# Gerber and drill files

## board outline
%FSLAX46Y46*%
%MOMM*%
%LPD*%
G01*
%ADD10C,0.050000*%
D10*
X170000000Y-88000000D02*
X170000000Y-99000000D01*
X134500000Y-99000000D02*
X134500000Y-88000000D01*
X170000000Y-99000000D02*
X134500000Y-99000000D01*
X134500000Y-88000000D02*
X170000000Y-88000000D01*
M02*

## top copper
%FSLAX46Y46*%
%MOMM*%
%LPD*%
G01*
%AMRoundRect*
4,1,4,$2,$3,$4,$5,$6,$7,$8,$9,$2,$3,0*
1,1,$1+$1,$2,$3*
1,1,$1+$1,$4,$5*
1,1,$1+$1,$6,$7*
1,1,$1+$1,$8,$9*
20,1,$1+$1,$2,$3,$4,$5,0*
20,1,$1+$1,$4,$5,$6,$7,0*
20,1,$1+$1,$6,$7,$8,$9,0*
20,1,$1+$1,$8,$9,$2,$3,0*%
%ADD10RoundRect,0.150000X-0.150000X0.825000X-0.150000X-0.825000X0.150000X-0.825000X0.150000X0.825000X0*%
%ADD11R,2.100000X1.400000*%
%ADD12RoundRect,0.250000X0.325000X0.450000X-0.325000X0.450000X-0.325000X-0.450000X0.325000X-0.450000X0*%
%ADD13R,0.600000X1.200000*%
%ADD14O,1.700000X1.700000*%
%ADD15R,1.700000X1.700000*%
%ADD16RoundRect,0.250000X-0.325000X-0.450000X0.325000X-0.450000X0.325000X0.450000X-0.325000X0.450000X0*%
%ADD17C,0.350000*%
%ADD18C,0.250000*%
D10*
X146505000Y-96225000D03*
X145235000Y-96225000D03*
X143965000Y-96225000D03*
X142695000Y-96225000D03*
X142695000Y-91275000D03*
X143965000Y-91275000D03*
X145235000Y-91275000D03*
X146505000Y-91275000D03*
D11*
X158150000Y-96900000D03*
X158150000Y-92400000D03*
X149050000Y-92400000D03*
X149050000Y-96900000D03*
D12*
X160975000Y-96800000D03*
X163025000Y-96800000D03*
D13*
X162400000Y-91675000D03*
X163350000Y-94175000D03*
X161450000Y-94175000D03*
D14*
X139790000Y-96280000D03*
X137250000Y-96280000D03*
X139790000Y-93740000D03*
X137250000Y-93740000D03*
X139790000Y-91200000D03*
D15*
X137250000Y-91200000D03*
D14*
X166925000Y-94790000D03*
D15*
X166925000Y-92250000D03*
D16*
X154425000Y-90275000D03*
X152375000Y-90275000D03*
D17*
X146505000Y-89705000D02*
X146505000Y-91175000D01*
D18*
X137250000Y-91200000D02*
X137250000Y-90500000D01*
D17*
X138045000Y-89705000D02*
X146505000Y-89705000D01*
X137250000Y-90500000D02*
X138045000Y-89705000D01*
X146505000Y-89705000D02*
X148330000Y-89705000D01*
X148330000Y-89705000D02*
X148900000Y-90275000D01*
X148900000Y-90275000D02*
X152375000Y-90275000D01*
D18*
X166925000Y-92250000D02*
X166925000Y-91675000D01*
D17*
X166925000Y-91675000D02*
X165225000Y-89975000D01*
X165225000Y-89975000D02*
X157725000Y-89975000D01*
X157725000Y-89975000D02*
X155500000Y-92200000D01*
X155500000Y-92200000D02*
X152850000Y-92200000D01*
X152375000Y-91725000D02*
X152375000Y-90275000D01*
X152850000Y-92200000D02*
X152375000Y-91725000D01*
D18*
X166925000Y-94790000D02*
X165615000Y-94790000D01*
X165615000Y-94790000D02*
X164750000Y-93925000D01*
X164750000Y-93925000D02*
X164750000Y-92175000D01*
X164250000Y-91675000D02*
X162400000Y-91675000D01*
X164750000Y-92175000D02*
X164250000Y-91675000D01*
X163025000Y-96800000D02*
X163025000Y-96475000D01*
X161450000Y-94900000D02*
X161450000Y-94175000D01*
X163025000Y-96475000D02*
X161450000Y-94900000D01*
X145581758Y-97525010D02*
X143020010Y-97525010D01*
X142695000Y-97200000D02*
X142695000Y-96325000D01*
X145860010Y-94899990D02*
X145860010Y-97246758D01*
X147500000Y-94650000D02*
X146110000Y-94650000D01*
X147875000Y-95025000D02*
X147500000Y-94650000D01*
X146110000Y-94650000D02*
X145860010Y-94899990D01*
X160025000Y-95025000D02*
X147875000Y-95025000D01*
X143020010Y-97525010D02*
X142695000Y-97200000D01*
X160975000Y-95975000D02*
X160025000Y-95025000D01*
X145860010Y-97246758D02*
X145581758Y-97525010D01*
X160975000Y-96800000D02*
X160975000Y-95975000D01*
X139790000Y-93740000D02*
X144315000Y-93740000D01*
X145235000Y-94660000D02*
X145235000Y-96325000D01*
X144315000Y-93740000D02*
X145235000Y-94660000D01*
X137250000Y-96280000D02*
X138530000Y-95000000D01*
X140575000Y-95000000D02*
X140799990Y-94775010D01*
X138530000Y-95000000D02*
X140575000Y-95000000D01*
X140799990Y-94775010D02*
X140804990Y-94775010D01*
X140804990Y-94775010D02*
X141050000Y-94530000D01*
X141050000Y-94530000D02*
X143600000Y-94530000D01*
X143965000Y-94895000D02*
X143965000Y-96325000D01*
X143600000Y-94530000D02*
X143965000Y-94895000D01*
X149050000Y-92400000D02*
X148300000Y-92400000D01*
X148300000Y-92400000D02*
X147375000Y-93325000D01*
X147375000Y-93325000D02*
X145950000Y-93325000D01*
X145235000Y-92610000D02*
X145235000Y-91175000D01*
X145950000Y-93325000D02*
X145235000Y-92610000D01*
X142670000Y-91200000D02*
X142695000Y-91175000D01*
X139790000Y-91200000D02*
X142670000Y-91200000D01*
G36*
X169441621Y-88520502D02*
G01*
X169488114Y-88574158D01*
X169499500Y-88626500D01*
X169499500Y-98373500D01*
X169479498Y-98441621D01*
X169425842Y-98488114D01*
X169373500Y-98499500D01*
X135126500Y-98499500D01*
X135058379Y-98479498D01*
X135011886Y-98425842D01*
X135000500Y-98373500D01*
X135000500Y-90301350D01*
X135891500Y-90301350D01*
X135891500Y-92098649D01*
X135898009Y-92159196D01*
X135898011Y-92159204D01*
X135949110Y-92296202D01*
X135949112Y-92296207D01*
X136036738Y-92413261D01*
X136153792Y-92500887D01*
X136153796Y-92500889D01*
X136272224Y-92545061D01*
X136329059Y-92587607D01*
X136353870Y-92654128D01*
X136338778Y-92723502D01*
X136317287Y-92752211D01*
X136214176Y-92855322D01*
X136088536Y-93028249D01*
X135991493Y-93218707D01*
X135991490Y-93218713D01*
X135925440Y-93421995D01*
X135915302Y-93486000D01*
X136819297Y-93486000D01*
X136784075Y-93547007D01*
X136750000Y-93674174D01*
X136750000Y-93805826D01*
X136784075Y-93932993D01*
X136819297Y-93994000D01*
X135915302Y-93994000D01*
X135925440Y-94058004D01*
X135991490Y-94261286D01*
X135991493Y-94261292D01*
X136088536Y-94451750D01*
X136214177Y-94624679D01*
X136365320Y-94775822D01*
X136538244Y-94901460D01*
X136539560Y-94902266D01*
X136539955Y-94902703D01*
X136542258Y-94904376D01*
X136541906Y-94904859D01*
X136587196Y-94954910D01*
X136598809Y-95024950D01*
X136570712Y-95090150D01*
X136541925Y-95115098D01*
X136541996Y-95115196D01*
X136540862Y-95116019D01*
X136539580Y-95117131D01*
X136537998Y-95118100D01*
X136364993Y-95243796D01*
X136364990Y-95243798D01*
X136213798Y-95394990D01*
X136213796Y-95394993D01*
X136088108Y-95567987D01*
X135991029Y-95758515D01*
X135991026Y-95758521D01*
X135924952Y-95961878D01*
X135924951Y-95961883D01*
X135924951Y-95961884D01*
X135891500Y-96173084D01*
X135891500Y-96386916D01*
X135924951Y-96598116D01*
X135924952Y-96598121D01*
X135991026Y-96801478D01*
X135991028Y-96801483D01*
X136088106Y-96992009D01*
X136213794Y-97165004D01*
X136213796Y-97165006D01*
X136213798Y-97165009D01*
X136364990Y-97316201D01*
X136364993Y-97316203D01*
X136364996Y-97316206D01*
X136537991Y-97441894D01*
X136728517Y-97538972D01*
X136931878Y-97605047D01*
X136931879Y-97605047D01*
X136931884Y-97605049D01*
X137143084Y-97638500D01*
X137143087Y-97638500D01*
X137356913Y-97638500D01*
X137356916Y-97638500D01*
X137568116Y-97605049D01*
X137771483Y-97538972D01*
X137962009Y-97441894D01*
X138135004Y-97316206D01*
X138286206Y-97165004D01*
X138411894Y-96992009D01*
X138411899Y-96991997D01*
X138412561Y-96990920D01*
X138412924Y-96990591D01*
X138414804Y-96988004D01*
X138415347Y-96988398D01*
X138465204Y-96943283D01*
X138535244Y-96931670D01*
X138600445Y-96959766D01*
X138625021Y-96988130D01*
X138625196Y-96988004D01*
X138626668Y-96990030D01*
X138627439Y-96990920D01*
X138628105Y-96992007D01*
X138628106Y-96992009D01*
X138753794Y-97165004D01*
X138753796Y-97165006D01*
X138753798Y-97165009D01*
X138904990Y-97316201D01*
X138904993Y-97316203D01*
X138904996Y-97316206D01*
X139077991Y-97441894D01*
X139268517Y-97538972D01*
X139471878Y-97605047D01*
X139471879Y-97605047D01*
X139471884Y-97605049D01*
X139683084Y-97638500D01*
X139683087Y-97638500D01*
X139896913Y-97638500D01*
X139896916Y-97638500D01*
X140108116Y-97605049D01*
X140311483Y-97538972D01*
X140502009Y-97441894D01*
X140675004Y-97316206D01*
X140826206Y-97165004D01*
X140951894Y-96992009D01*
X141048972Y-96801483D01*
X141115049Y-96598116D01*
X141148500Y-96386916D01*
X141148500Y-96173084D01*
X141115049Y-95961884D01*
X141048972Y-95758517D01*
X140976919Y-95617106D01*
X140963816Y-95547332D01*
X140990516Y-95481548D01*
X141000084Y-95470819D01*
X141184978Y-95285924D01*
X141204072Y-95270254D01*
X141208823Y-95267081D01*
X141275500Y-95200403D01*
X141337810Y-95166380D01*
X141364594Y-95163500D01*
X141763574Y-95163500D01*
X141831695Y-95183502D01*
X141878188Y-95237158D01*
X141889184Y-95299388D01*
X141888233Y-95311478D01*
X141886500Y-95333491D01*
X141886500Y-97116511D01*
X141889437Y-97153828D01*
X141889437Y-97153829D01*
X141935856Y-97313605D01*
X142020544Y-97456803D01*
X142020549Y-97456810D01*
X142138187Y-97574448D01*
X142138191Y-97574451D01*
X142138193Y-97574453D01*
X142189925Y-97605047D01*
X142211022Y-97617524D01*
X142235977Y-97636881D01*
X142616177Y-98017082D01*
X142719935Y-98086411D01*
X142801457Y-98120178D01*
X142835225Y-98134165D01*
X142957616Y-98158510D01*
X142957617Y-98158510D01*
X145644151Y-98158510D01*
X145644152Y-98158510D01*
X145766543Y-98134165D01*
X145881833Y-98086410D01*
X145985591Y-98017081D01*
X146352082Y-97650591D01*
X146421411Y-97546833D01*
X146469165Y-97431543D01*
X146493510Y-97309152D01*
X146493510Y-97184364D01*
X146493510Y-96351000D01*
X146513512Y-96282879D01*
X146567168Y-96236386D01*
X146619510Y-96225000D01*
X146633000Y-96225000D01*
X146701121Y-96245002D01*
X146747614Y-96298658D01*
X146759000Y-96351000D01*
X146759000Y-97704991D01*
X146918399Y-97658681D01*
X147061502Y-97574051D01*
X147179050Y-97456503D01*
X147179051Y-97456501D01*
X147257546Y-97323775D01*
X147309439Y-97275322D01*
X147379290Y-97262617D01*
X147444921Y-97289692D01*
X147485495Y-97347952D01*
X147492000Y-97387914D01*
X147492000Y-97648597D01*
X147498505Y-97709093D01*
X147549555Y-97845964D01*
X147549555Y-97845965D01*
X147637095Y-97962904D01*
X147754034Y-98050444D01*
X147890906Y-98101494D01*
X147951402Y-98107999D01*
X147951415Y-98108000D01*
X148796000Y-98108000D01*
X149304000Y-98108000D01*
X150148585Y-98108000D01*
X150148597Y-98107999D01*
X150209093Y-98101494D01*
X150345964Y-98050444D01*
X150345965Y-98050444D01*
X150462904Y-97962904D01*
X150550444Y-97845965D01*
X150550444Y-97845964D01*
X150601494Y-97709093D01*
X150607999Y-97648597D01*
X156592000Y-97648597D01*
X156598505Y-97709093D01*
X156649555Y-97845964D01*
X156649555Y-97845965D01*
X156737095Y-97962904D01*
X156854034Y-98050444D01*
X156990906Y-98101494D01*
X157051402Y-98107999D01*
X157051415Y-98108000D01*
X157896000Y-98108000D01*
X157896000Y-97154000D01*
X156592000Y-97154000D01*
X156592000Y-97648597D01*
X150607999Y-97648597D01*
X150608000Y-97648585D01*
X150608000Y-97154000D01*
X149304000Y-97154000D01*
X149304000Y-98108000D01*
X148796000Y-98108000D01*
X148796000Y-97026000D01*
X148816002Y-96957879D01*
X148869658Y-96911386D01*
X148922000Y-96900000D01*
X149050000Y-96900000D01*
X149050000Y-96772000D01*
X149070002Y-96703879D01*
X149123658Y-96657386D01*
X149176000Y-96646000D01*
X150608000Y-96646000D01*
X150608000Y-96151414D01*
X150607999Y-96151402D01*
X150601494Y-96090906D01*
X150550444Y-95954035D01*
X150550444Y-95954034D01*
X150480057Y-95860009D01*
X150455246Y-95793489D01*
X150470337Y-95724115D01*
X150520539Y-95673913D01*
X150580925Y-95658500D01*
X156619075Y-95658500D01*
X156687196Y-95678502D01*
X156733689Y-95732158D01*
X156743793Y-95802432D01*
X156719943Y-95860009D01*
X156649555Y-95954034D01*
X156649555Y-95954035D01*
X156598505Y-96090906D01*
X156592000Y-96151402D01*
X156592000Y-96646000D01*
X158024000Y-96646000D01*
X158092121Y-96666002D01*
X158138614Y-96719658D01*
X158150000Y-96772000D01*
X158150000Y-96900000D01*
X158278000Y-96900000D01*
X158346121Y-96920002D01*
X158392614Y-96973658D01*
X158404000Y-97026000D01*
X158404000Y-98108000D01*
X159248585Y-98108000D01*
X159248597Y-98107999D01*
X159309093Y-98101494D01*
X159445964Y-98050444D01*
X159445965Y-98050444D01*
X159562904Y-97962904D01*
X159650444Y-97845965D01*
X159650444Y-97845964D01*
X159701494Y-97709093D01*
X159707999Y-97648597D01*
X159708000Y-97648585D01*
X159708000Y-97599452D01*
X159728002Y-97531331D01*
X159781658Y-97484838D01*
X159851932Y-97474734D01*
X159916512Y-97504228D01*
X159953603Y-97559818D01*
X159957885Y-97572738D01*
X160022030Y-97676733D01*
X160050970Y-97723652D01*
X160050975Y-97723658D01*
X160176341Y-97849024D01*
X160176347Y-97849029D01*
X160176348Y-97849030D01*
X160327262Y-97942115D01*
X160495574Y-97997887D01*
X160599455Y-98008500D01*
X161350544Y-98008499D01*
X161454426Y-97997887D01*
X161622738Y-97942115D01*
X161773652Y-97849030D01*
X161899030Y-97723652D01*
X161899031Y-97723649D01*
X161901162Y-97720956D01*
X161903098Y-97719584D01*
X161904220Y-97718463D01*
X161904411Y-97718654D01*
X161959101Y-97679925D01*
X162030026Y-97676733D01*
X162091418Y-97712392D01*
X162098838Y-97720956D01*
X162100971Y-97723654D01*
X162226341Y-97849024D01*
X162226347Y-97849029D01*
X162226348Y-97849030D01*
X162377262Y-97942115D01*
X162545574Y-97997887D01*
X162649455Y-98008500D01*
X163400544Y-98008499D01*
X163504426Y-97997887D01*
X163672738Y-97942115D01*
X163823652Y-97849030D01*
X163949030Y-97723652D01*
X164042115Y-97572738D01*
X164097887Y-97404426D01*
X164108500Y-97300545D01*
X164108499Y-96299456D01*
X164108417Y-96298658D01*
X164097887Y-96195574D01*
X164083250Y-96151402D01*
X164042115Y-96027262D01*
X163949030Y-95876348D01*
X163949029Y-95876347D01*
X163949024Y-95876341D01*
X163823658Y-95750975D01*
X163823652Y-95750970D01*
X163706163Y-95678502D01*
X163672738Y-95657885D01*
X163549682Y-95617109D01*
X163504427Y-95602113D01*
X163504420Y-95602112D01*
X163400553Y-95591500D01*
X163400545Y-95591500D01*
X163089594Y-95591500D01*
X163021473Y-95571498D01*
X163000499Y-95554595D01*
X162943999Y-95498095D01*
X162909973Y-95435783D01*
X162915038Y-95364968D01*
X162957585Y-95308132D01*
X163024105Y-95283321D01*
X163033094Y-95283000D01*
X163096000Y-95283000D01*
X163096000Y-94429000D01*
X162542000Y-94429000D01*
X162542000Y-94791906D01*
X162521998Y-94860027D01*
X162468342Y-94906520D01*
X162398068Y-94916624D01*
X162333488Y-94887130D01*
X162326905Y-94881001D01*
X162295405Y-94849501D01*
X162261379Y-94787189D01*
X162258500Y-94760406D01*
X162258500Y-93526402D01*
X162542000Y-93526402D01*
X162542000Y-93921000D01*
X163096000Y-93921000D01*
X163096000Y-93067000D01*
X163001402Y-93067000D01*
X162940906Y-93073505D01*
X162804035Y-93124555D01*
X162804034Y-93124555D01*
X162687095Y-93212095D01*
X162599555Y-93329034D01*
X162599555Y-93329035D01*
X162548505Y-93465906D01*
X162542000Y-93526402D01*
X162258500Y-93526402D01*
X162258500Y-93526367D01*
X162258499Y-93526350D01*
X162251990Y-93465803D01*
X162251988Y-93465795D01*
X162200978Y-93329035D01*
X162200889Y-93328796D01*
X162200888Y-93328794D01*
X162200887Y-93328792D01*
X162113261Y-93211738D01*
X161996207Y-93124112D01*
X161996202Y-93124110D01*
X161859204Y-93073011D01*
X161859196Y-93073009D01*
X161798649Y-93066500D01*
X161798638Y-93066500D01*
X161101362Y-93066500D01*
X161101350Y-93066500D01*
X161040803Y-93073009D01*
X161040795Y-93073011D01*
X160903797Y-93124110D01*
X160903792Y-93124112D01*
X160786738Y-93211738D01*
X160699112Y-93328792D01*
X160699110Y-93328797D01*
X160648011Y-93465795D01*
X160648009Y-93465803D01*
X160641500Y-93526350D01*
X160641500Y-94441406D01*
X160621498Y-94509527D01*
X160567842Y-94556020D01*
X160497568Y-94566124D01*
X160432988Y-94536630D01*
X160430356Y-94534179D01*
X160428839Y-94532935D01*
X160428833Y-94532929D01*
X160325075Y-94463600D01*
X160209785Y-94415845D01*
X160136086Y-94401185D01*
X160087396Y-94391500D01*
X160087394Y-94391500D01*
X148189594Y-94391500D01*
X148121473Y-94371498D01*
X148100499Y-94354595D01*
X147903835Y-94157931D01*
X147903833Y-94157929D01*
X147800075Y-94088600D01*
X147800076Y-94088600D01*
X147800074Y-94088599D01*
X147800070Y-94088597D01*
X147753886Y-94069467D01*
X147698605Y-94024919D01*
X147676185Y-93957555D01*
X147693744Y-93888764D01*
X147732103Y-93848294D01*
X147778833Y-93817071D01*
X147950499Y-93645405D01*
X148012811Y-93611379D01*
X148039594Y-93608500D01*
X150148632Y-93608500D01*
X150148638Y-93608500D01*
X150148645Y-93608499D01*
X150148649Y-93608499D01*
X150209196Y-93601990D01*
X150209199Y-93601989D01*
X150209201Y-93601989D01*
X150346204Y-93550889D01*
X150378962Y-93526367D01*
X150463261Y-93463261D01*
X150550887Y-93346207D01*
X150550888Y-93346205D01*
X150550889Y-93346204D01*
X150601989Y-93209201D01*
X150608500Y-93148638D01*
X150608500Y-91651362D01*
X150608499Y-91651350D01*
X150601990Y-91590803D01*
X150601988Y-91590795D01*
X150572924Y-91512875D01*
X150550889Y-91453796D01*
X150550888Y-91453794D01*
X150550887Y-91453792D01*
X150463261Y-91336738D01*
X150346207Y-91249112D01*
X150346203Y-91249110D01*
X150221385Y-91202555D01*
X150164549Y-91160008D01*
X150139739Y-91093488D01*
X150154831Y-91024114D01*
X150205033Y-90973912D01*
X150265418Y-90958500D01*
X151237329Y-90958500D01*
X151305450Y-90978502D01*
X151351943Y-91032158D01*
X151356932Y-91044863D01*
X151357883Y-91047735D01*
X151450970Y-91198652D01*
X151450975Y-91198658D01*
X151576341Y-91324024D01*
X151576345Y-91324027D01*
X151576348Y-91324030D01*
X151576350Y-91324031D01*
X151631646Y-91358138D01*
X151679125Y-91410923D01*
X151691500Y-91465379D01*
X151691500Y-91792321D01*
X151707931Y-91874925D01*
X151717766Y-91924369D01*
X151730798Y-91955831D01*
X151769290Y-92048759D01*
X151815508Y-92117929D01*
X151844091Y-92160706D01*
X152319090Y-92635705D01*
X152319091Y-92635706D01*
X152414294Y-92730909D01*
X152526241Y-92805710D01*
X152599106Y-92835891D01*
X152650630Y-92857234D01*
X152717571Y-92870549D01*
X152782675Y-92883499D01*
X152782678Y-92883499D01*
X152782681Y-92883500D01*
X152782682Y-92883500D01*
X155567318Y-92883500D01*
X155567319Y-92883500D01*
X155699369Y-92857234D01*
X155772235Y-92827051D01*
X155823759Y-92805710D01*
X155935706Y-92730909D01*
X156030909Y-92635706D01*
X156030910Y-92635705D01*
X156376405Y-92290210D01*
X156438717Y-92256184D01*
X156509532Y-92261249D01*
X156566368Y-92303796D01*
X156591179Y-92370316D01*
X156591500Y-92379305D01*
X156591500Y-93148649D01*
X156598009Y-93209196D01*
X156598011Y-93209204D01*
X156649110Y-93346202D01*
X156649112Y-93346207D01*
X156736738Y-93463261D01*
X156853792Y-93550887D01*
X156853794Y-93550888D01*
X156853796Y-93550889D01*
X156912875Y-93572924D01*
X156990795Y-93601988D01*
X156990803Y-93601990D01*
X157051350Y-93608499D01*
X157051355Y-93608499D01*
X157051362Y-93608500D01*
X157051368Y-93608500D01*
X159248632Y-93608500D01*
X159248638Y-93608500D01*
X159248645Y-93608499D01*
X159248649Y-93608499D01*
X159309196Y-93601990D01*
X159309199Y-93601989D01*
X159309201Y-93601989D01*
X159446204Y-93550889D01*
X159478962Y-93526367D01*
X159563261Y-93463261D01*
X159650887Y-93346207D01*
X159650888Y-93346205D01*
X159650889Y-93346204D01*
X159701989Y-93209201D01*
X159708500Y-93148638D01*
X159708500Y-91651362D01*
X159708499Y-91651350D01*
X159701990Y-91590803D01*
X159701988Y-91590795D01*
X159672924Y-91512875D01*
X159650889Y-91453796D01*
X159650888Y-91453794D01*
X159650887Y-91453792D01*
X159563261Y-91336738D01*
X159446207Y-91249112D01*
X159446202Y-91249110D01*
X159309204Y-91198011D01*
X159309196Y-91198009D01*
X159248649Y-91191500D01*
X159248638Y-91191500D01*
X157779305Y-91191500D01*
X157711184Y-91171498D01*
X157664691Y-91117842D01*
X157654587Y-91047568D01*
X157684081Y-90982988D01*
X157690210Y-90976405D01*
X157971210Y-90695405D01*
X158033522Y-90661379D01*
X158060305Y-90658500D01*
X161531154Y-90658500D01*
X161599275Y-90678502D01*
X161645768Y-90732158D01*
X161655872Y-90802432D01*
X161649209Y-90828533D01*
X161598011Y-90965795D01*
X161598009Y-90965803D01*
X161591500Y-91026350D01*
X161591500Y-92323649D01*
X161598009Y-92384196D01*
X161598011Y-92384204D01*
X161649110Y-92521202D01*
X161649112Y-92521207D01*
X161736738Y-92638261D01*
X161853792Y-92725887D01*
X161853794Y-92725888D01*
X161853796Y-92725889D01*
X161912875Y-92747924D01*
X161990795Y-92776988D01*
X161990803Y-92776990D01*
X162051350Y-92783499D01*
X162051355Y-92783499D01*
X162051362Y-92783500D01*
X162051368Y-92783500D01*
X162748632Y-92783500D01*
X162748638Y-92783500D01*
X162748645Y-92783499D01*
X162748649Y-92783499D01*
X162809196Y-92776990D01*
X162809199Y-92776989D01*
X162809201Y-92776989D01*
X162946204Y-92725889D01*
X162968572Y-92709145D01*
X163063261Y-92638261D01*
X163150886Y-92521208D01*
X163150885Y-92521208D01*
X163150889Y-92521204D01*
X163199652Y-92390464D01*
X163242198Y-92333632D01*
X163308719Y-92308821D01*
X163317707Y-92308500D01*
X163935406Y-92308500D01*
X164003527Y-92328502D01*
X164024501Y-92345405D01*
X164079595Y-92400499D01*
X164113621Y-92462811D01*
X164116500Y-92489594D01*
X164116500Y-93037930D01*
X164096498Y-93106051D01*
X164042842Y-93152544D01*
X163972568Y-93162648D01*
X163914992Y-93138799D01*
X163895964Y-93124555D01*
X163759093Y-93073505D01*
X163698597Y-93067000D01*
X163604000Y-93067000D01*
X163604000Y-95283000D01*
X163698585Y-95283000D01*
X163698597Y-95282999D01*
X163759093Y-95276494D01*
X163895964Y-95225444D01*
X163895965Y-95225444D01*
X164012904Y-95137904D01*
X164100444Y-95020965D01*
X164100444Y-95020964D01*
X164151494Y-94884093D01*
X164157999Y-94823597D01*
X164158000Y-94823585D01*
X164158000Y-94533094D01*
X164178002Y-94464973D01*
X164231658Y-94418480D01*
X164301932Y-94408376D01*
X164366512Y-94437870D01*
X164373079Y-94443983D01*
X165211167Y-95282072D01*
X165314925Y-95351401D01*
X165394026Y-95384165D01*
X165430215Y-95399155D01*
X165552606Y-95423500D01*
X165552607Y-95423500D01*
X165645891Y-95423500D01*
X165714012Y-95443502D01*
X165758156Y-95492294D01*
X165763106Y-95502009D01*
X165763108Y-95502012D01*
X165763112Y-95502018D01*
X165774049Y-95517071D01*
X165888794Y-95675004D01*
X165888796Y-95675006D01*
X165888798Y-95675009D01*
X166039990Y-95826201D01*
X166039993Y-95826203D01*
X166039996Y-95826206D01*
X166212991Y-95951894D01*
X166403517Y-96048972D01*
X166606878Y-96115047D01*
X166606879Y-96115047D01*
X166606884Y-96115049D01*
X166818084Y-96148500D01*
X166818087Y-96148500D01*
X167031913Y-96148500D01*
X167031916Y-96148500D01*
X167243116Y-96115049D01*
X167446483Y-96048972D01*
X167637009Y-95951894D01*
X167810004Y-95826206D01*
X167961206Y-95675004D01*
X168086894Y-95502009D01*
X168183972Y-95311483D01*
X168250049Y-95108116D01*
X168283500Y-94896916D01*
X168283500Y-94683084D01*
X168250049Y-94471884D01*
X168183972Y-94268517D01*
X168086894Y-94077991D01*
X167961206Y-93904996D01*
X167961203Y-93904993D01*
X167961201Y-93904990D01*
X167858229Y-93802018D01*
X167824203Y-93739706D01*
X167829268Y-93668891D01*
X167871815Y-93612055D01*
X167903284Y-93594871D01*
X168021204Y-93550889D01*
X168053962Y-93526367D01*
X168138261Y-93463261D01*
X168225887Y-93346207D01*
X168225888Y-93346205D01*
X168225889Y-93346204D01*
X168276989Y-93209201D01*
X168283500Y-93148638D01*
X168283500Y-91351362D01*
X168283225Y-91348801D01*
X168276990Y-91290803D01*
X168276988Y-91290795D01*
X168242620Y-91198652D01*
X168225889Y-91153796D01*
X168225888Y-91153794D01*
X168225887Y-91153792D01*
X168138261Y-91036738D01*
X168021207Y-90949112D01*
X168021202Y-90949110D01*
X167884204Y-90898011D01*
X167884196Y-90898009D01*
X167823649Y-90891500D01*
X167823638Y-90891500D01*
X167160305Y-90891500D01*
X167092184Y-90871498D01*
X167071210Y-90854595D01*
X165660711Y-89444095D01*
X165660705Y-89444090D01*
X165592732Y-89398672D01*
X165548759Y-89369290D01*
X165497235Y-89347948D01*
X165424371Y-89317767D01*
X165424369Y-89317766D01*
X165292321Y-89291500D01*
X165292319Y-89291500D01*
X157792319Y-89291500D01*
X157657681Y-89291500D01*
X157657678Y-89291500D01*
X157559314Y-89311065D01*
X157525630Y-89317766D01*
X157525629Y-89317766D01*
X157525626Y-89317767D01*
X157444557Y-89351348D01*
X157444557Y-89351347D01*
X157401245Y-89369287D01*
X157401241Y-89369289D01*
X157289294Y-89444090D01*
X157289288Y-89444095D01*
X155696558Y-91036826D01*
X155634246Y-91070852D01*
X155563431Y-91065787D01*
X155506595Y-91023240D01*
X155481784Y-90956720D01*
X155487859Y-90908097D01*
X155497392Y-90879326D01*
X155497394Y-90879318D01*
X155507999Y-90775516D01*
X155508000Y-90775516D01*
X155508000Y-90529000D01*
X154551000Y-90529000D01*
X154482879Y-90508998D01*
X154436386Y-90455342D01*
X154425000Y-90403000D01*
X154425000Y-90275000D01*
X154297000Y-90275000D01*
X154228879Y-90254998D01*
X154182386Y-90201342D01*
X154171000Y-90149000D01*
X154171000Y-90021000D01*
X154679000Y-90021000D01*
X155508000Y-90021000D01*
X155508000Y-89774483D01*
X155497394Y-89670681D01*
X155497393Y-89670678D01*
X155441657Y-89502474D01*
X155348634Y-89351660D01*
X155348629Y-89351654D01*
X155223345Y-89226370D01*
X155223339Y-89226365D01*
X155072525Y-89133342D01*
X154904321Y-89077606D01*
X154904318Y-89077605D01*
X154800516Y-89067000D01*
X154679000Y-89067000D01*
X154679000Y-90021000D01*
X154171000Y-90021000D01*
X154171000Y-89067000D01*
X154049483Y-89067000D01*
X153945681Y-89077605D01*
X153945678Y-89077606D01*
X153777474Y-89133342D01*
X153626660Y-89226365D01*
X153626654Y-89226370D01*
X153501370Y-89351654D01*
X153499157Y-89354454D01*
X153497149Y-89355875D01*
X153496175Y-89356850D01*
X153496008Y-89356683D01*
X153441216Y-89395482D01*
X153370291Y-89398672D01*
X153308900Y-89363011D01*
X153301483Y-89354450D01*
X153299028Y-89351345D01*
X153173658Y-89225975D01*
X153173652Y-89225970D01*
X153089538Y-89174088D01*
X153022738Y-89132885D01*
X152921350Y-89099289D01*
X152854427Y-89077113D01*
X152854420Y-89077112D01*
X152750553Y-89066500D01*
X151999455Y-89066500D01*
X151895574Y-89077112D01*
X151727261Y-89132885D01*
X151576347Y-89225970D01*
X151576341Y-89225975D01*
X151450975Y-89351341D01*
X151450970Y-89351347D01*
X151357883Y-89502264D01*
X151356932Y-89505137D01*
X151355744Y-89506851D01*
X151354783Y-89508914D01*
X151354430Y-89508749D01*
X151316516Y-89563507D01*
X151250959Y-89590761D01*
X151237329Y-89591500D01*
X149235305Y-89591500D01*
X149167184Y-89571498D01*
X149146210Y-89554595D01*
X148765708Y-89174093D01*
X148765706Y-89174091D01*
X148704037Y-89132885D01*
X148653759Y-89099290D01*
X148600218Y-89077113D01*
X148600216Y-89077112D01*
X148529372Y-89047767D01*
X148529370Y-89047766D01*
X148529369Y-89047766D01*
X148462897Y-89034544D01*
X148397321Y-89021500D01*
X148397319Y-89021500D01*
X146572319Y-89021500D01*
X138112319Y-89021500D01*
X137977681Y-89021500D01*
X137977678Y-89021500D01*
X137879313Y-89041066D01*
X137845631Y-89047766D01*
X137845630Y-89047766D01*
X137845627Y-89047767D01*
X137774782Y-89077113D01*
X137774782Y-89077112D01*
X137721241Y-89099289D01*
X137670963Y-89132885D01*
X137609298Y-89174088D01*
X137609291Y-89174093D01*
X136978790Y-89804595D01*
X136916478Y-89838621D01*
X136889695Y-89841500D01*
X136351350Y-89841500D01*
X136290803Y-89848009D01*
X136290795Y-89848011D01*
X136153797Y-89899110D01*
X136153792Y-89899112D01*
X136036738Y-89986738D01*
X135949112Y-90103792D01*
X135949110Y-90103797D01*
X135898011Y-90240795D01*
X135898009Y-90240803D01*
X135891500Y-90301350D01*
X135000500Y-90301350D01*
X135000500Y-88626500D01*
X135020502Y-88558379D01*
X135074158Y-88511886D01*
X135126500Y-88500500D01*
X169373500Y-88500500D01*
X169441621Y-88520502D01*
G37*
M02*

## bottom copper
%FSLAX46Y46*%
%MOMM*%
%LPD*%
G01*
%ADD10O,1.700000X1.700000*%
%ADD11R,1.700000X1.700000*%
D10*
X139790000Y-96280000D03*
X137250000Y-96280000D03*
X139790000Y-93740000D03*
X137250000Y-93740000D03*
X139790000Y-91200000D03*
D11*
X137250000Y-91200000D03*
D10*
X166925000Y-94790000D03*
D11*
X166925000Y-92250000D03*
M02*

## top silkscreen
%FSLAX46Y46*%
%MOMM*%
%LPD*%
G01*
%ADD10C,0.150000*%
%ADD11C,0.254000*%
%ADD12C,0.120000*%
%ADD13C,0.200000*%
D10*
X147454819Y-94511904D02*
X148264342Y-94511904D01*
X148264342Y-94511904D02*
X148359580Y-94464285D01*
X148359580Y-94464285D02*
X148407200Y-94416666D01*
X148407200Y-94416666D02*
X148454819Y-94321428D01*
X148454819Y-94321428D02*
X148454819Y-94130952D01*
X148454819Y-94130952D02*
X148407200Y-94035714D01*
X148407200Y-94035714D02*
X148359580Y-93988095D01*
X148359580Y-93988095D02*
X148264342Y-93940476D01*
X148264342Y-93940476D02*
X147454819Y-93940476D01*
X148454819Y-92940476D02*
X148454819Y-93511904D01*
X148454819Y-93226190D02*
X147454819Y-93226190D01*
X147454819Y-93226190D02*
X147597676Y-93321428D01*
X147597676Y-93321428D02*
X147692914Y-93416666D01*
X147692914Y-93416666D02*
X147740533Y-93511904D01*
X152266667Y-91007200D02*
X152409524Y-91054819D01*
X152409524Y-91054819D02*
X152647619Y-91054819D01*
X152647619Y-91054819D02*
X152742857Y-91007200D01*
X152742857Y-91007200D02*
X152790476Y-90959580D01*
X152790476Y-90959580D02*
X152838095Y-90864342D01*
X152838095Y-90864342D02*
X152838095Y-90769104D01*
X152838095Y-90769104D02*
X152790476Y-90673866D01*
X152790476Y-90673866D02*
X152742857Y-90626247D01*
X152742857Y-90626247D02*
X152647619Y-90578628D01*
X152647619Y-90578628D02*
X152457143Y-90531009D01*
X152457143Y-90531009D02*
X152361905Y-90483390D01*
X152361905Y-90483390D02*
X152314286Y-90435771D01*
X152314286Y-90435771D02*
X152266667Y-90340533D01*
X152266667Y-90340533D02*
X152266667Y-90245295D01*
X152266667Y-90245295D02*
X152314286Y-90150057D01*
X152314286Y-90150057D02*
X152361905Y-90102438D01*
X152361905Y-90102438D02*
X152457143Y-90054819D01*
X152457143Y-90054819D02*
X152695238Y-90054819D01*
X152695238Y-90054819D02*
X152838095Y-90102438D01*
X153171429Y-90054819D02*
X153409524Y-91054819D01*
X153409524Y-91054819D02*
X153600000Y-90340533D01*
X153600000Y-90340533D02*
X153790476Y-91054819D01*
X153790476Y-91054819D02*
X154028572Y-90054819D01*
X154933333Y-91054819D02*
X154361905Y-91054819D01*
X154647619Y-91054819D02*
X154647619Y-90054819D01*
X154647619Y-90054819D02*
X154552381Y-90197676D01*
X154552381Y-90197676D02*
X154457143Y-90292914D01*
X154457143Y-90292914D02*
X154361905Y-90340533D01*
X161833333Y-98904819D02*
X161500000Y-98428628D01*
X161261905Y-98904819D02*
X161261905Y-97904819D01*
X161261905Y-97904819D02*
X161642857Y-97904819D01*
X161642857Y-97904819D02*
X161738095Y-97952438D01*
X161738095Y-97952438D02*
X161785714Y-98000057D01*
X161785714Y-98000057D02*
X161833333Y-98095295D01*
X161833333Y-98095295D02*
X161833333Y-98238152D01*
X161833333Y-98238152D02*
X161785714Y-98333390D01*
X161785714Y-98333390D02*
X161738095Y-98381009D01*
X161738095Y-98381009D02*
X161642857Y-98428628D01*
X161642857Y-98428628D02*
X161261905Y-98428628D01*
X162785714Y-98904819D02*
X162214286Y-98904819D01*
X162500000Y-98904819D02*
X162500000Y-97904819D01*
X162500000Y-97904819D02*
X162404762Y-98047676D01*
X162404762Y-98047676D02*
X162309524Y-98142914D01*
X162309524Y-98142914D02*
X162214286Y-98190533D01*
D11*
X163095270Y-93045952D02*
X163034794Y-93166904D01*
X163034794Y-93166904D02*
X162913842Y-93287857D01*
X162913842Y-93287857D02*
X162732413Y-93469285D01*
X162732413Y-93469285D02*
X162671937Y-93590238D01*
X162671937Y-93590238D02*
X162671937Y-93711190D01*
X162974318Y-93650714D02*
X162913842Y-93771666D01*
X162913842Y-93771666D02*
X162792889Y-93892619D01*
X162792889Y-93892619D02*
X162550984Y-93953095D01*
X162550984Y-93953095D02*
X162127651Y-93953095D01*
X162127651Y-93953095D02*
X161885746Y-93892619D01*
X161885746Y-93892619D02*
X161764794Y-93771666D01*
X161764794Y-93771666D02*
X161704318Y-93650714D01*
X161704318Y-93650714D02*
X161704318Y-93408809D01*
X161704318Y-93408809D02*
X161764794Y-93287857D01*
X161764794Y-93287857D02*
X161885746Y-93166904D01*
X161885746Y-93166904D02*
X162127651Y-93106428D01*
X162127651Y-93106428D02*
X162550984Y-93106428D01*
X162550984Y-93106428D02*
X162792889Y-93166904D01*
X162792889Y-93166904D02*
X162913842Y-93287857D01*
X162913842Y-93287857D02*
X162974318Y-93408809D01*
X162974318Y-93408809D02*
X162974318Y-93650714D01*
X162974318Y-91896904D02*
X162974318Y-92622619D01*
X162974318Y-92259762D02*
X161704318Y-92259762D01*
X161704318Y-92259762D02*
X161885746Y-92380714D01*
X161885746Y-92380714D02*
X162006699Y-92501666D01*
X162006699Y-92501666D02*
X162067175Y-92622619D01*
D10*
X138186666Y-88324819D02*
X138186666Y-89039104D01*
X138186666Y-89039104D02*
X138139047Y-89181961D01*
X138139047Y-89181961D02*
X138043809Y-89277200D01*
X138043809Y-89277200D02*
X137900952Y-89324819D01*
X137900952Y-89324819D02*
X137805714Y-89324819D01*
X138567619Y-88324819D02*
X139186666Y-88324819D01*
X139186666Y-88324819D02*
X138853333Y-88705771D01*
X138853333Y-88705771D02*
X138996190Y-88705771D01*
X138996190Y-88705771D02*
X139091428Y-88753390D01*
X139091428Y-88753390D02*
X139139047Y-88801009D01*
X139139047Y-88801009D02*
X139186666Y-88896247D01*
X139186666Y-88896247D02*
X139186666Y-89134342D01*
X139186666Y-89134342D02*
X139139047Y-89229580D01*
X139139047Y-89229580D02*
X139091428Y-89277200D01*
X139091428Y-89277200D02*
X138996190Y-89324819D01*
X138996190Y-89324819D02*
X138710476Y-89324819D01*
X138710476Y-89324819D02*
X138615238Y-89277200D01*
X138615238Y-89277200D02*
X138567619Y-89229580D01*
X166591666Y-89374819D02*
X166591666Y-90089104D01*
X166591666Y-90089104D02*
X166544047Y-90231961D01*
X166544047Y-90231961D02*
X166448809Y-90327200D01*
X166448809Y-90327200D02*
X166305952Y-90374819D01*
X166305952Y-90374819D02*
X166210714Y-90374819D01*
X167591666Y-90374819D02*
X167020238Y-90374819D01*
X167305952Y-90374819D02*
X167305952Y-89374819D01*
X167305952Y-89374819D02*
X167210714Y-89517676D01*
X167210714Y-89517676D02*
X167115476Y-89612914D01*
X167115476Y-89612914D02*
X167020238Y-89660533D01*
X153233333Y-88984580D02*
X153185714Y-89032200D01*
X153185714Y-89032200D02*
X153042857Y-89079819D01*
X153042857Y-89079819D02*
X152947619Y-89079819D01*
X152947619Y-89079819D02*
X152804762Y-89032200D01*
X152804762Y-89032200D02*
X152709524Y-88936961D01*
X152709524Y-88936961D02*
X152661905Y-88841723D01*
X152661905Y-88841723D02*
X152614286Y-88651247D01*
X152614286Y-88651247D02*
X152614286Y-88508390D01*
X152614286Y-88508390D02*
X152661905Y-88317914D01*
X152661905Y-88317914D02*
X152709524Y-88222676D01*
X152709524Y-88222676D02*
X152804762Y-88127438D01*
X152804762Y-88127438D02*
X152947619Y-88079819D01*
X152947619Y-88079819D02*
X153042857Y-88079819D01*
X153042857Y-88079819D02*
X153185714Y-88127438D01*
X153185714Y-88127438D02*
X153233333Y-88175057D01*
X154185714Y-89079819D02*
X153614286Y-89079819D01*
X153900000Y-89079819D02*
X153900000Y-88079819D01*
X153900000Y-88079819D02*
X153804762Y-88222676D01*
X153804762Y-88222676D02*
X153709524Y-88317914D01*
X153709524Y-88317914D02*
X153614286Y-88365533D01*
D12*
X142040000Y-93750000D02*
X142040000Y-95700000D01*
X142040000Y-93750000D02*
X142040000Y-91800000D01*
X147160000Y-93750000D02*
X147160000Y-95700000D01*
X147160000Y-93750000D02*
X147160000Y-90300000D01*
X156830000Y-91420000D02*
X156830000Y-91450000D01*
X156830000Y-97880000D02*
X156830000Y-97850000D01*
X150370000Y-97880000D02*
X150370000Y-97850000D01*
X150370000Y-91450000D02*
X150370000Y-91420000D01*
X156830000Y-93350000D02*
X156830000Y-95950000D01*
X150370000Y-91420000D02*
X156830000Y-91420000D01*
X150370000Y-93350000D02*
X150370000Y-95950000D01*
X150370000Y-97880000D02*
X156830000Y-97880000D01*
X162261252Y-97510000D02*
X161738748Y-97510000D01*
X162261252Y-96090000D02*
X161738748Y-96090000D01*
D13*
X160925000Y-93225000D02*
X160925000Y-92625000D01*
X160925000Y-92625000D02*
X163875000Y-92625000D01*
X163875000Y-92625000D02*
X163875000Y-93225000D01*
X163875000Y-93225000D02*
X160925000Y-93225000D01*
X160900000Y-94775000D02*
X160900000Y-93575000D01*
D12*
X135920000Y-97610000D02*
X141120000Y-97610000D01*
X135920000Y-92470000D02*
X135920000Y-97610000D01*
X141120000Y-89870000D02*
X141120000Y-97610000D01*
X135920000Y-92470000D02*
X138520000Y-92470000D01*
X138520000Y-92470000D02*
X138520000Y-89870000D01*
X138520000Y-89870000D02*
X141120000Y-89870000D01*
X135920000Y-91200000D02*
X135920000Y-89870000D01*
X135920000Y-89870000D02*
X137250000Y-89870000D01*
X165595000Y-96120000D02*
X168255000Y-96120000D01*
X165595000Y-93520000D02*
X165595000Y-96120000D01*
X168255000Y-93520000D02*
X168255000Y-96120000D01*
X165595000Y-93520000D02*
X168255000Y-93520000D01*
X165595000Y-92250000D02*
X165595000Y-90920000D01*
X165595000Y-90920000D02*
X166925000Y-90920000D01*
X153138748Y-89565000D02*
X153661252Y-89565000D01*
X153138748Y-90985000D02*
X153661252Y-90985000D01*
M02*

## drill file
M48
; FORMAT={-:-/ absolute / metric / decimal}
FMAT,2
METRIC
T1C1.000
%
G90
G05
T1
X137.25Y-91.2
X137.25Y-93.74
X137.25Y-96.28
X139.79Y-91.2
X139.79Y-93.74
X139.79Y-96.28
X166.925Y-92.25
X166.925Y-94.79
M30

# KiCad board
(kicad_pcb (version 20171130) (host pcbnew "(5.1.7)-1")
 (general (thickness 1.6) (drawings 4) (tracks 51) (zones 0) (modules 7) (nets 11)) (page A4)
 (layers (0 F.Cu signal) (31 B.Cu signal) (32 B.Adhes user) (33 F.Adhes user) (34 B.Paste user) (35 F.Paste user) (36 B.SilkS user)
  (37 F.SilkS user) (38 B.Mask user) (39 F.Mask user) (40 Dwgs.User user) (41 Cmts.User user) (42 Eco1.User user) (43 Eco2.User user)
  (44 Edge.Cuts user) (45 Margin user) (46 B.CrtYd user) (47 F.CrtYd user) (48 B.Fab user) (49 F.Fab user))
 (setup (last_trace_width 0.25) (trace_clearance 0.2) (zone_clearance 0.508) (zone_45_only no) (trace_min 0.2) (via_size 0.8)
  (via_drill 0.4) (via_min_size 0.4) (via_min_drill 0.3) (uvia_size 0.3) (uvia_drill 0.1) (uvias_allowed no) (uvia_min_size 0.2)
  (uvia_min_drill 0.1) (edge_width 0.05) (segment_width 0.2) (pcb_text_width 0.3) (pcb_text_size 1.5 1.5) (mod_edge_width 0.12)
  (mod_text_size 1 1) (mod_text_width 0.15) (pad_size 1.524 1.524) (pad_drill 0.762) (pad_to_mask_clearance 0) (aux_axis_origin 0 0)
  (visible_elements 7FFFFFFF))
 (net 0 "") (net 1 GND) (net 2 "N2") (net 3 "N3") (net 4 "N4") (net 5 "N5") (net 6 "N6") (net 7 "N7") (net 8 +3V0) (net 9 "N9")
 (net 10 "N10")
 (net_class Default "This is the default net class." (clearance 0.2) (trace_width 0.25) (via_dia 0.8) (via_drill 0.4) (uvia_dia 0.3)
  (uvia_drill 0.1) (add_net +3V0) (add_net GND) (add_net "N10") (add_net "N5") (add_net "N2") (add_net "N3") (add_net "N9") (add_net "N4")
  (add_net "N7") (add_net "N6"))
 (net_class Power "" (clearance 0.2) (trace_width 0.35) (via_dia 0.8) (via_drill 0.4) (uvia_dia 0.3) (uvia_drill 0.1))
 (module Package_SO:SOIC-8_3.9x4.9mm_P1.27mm (layer F.Cu) (at 144.6 93.75 270)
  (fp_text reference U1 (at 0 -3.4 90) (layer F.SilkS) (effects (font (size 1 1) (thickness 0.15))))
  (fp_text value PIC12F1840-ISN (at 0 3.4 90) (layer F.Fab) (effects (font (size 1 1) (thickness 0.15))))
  (fp_line (start 0 2.56) (end 1.95 2.56) (layer F.SilkS) (width 0.12))
  (fp_line (start 0 2.56) (end -1.95 2.56) (layer F.SilkS) (width 0.12))
  (fp_line (start 0 -2.56) (end 1.95 -2.56) (layer F.SilkS) (width 0.12))
  (fp_line (start 0 -2.56) (end -3.45 -2.56) (layer F.SilkS) (width 0.12))
  (pad 8 smd roundrect (at 2.475 -1.905 270) (size 1.95 0.6) (layers F.Cu F.Paste F.Mask) (roundrect_rratio 0.25) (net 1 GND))
  (pad 7 smd roundrect (at 2.475 -0.635 270) (size 1.95 0.6) (layers F.Cu F.Paste F.Mask) (roundrect_rratio 0.25) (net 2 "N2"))
  (pad 6 smd roundrect (at 2.475 0.635 270) (size 1.95 0.6) (layers F.Cu F.Paste F.Mask) (roundrect_rratio 0.25) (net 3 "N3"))
  (pad 5 smd roundrect (at 2.475 1.905 270) (size 1.95 0.6) (layers F.Cu F.Paste F.Mask) (roundrect_rratio 0.25) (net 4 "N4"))
  (pad 4 smd roundrect (at -2.475 1.905 270) (size 1.95 0.6) (layers F.Cu F.Paste F.Mask) (roundrect_rratio 0.25) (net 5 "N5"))
  (pad 3 smd roundrect (at -2.475 0.635 270) (size 1.95 0.6) (layers F.Cu F.Paste F.Mask) (roundrect_rratio 0.25) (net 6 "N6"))
  (pad 2 smd roundrect (at -2.475 -0.635 270) (size 1.95 0.6) (layers F.Cu F.Paste F.Mask) (roundrect_rratio 0.25) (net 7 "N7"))
  (pad 1 smd roundrect (at -2.475 -1.905 270) (size 1.95 0.6) (layers F.Cu F.Paste F.Mask) (roundrect_rratio 0.25) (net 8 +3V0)))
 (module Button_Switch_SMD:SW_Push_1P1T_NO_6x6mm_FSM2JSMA (layer F.Cu) (at 153.6 94.65)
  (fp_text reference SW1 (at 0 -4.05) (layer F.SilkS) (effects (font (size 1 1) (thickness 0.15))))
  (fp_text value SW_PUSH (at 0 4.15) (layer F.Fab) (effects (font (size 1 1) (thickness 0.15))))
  (fp_line (start 3.23 -3.23) (end 3.23 -3.2) (layer F.SilkS) (width 0.12))
  (fp_line (start 3.23 3.23) (end 3.23 3.2) (layer F.SilkS) (width 0.12))
  (fp_line (start -3.23 3.23) (end -3.23 3.2) (layer F.SilkS) (width 0.12))
  (fp_line (start -3.23 -3.2) (end -3.23 -3.23) (layer F.SilkS) (width 0.12))
  (fp_line (start 3.23 -1.3) (end 3.23 1.3) (layer F.SilkS) (width 0.12))
  (fp_line (start -3.23 -3.23) (end 3.23 -3.23) (layer F.SilkS) (width 0.12))
  (fp_line (start -3.23 -1.3) (end -3.23 1.3) (layer F.SilkS) (width 0.12))
  (fp_line (start -3.23 3.23) (end 3.23 3.23) (layer F.SilkS) (width 0.12))
  (pad 2 smd rect (at 4.55 2.25) (size 2.1 1.4) (layers F.Cu F.Paste F.Mask) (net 1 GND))
  (pad 1 smd rect (at 4.55 -2.25) (size 2.1 1.4) (layers F.Cu F.Paste F.Mask) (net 7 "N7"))
  (pad 1 smd rect (at -4.55 -2.25) (size 2.1 1.4) (layers F.Cu F.Paste F.Mask) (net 7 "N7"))
  (pad 2 smd rect (at -4.55 2.25) (size 2.1 1.4) (layers F.Cu F.Paste F.Mask) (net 1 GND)))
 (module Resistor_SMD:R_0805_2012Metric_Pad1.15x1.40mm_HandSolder (layer F.Cu) (at 162 96.8 180)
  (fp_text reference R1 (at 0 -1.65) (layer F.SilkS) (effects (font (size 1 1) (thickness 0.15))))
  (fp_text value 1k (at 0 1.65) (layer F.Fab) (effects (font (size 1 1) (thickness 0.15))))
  (fp_line (start -0.261252 -0.71) (end 0.261252 -0.71) (layer F.SilkS) (width 0.12))
  (fp_line (start -0.261252 0.71) (end 0.261252 0.71) (layer F.SilkS) (width 0.12))
  (pad 2 smd roundrect (at 1.025 0 180) (size 1.15 1.4) (layers F.Cu F.Paste F.Mask) (roundrect_rratio 0.217391) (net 4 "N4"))
  (pad 1 smd roundrect (at -1.025 0 180) (size 1.15 1.4) (layers F.Cu F.Paste F.Mask) (roundrect_rratio 0.217391) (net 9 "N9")))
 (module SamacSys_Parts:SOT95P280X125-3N (layer F.Cu) (at 162.4 92.925 90)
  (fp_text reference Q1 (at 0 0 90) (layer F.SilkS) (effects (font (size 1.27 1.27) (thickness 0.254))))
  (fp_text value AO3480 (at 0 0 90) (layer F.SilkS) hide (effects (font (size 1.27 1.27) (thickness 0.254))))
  (fp_line (start -0.3 -1.475) (end 0.3 -1.475) (layer F.SilkS) (width 0.2))
  (fp_line (start 0.3 -1.475) (end 0.3 1.475) (layer F.SilkS) (width 0.2))
  (fp_line (start 0.3 1.475) (end -0.3 1.475) (layer F.SilkS) (width 0.2))
  (fp_line (start -0.3 1.475) (end -0.3 -1.475) (layer F.SilkS) (width 0.2))
  (fp_line (start -1.85 -1.5) (end -0.65 -1.5) (layer F.SilkS) (width 0.2))
  (pad 3 smd rect (at 1.25 0 180) (size 0.6 1.2) (layers F.Cu F.Paste F.Mask) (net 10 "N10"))
  (pad 2 smd rect (at -1.25 0.95 180) (size 0.6 1.2) (layers F.Cu F.Paste F.Mask) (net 1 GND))
  (pad 1 smd rect (at -1.25 -0.95 180) (size 0.6 1.2) (layers F.Cu F.Paste F.Mask) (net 9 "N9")))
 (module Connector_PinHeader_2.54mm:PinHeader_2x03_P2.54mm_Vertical (layer F.Cu) (at 137.25 91.2)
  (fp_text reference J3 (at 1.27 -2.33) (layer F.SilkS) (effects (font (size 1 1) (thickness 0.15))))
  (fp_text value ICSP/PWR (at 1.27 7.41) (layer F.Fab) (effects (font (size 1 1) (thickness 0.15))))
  (fp_line (start -1.33 6.41) (end 3.87 6.41) (layer F.SilkS) (width 0.12))
  (fp_line (start -1.33 1.27) (end -1.33 6.41) (layer F.SilkS) (width 0.12))
  (fp_line (start 3.87 -1.33) (end 3.87 6.41) (layer F.SilkS) (width 0.12))
  (fp_line (start -1.33 1.27) (end 1.27 1.27) (layer F.SilkS) (width 0.12))
  (fp_line (start 1.27 1.27) (end 1.27 -1.33) (layer F.SilkS) (width 0.12))
  (fp_line (start 1.27 -1.33) (end 3.87 -1.33) (layer F.SilkS) (width 0.12))
  (fp_line (start -1.33 0) (end -1.33 -1.33) (layer F.SilkS) (width 0.12))
  (fp_line (start -1.33 -1.33) (end 0 -1.33) (layer F.SilkS) (width 0.12))
  (pad 6 thru_hole oval (at 2.54 5.08) (size 1.7 1.7) (drill 1) (layers *.Cu *.Mask))
  (pad 5 thru_hole oval (at 0 5.08) (size 1.7 1.7) (drill 1) (layers *.Cu *.Mask) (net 3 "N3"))
  (pad 4 thru_hole oval (at 2.54 2.54) (size 1.7 1.7) (drill 1) (layers *.Cu *.Mask) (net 2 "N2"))
  (pad 3 thru_hole oval (at 0 2.54) (size 1.7 1.7) (drill 1) (layers *.Cu *.Mask) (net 1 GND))
  (pad 2 thru_hole oval (at 2.54 0) (size 1.7 1.7) (drill 1) (layers *.Cu *.Mask) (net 5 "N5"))
  (pad 1 thru_hole rect (at 0 0) (size 1.7 1.7) (drill 1) (layers *.Cu *.Mask) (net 8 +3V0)))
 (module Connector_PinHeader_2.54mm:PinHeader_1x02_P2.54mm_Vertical (layer F.Cu) (at 166.925 92.25)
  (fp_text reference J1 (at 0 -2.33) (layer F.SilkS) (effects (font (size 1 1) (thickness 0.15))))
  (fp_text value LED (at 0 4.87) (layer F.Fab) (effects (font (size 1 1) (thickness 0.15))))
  (fp_line (start -1.33 3.87) (end 1.33 3.87) (layer F.SilkS) (width 0.12))
  (fp_line (start -1.33 1.27) (end -1.33 3.87) (layer F.SilkS) (width 0.12))
  (fp_line (start 1.33 1.27) (end 1.33 3.87) (layer F.SilkS) (width 0.12))
  (fp_line (start -1.33 1.27) (end 1.33 1.27) (layer F.SilkS) (width 0.12))
  (fp_line (start -1.33 0) (end -1.33 -1.33) (layer F.SilkS) (width 0.12))
  (fp_line (start -1.33 -1.33) (end 0 -1.33) (layer F.SilkS) (width 0.12))
  (pad 2 thru_hole oval (at 0 2.54) (size 1.7 1.7) (drill 1) (layers *.Cu *.Mask) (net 10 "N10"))
  (pad 1 thru_hole rect (at 0 0) (size 1.7 1.7) (drill 1) (layers *.Cu *.Mask) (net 8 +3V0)))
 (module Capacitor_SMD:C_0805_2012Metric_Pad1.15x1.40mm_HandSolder (layer F.Cu) (at 153.4 90.275)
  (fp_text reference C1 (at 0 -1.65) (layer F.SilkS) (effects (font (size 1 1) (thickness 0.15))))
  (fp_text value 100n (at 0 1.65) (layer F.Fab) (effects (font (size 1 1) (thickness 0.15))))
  (fp_line (start -0.261252 -0.71) (end 0.261252 -0.71) (layer F.SilkS) (width 0.12))
  (fp_line (start -0.261252 0.71) (end 0.261252 0.71) (layer F.SilkS) (width 0.12))
  (pad 2 smd roundrect (at 1.025 0) (size 1.15 1.4) (layers F.Cu F.Paste F.Mask) (roundrect_rratio 0.217391) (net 1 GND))
  (pad 1 smd roundrect (at -1.025 0) (size 1.15 1.4) (layers F.Cu F.Paste F.Mask) (roundrect_rratio 0.217391) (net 8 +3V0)))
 (gr_line (start 170 88) (end 170 99) (layer Edge.Cuts) (width 0.05))
 (gr_line (start 134.5 99) (end 134.5 88) (layer Edge.Cuts) (width 0.05))
 (gr_line (start 170 99) (end 134.5 99) (layer Edge.Cuts) (width 0.05))
 (gr_line (start 134.5 88) (end 170 88) (layer Edge.Cuts) (width 0.05))
 (segment (start 146.505 89.705) (end 146.505 91.175) (width 0.35) (layer F.Cu) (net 8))
 (segment (start 137.25 91.2) (end 137.25 90.5) (width 0.25) (layer F.Cu) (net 8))
 (segment (start 138.045 89.705) (end 146.505 89.705) (width 0.35) (layer F.Cu) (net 8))
 (segment (start 137.25 90.5) (end 138.045 89.705) (width 0.35) (layer F.Cu) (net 8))
 (segment (start 146.505 89.705) (end 148.33 89.705) (width 0.35) (layer F.Cu) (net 8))
 (segment (start 148.33 89.705) (end 148.9 90.275) (width 0.35) (layer F.Cu) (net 8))
 (segment (start 148.9 90.275) (end 152.375 90.275) (width 0.35) (layer F.Cu) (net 8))
 (segment (start 166.925 92.25) (end 166.925 91.675) (width 0.25) (layer F.Cu) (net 8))
 (segment (start 166.925 91.675) (end 165.225 89.975) (width 0.35) (layer F.Cu) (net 8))
 (segment (start 165.225 89.975) (end 157.725 89.975) (width 0.35) (layer F.Cu) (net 8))
 (segment (start 157.725 89.975) (end 155.5 92.2) (width 0.35) (layer F.Cu) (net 8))
 (segment (start 155.5 92.2) (end 152.85 92.2) (width 0.35) (layer F.Cu) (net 8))
 (segment (start 152.375 91.725) (end 152.375 90.275) (width 0.35) (layer F.Cu) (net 8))
 (segment (start 152.85 92.2) (end 152.375 91.725) (width 0.35) (layer F.Cu) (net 8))
 (segment (start 166.925 94.79) (end 165.615 94.79) (width 0.25) (layer F.Cu) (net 10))
 (segment (start 165.615 94.79) (end 164.75 93.925) (width 0.25) (layer F.Cu) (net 10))
 (segment (start 164.75 93.925) (end 164.75 92.175) (width 0.25) (layer F.Cu) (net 10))
 (segment (start 164.25 91.675) (end 162.4 91.675) (width 0.25) (layer F.Cu) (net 10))
 (segment (start 164.75 92.175) (end 164.25 91.675) (width 0.25) (layer F.Cu) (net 10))
 (segment (start 163.025 96.8) (end 163.025 96.475) (width 0.25) (layer F.Cu) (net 9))
 (segment (start 161.45 94.9) (end 161.45 94.175) (width 0.25) (layer F.Cu) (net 9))
 (segment (start 163.025 96.475) (end 161.45 94.9) (width 0.25) (layer F.Cu) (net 9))
 (segment (start 145.581758 97.52501) (end 143.02001 97.52501) (width 0.25) (layer F.Cu) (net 4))
 (segment (start 142.695 97.2) (end 142.695 96.325) (width 0.25) (layer F.Cu) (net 4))
 (segment (start 145.86001 94.89999) (end 145.86001 97.246758) (width 0.25) (layer F.Cu) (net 4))
 (segment (start 147.5 94.65) (end 146.11 94.65) (width 0.25) (layer F.Cu) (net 4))
 (segment (start 147.875 95.025) (end 147.5 94.65) (width 0.25) (layer F.Cu) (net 4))
 (segment (start 146.11 94.65) (end 145.86001 94.89999) (width 0.25) (layer F.Cu) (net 4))
 (segment (start 160.025 95.025) (end 147.875 95.025) (width 0.25) (layer F.Cu) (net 4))
 (segment (start 143.02001 97.52501) (end 142.695 97.2) (width 0.25) (layer F.Cu) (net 4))
 (segment (start 160.975 95.975) (end 160.025 95.025) (width 0.25) (layer F.Cu) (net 4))
 (segment (start 145.86001 97.246758) (end 145.581758 97.52501) (width 0.25) (layer F.Cu) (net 4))
 (segment (start 160.975 96.8) (end 160.975 95.975) (width 0.25) (layer F.Cu) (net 4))
 (segment (start 139.79 93.74) (end 144.315 93.74) (width 0.25) (layer F.Cu) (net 2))
 (segment (start 145.235 94.66) (end 145.235 96.325) (width 0.25) (layer F.Cu) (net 2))
 (segment (start 144.315 93.74) (end 145.235 94.66) (width 0.25) (layer F.Cu) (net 2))
 (segment (start 137.25 96.28) (end 138.53 95) (width 0.25) (layer F.Cu) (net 3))
 (segment (start 140.575 95) (end 140.79999 94.77501) (width 0.25) (layer F.Cu) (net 3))
 (segment (start 138.53 95) (end 140.575 95) (width 0.25) (layer F.Cu) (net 3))
 (segment (start 140.79999 94.77501) (end 140.80499 94.77501) (width 0.25) (layer F.Cu) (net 3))
 (segment (start 140.80499 94.77501) (end 141.05 94.53) (width 0.25) (layer F.Cu) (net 3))
 (segment (start 141.05 94.53) (end 143.6 94.53) (width 0.25) (layer F.Cu) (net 3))
 (segment (start 143.965 94.895) (end 143.965 96.325) (width 0.25) (layer F.Cu) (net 3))
 (segment (start 143.6 94.53) (end 143.965 94.895) (width 0.25) (layer F.Cu) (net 3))
 (segment (start 149.05 92.4) (end 148.3 92.4) (width 0.25) (layer F.Cu) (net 7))
 (segment (start 148.3 92.4) (end 147.375 93.325) (width 0.25) (layer F.Cu) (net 7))
 (segment (start 147.375 93.325) (end 145.95 93.325) (width 0.25) (layer F.Cu) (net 7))
 (segment (start 145.235 92.61) (end 145.235 91.175) (width 0.25) (layer F.Cu) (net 7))
 (segment (start 145.95 93.325) (end 145.235 92.61) (width 0.25) (layer F.Cu) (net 7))
 (segment (start 142.67 91.2) (end 142.695 91.175) (width 0.25) (layer F.Cu) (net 5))
 (segment (start 139.79 91.2) (end 142.67 91.2) (width 0.25) (layer F.Cu) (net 5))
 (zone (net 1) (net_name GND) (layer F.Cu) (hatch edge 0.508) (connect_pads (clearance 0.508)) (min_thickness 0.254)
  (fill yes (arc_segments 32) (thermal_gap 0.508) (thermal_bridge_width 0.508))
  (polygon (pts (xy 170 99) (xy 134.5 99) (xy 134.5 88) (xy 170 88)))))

